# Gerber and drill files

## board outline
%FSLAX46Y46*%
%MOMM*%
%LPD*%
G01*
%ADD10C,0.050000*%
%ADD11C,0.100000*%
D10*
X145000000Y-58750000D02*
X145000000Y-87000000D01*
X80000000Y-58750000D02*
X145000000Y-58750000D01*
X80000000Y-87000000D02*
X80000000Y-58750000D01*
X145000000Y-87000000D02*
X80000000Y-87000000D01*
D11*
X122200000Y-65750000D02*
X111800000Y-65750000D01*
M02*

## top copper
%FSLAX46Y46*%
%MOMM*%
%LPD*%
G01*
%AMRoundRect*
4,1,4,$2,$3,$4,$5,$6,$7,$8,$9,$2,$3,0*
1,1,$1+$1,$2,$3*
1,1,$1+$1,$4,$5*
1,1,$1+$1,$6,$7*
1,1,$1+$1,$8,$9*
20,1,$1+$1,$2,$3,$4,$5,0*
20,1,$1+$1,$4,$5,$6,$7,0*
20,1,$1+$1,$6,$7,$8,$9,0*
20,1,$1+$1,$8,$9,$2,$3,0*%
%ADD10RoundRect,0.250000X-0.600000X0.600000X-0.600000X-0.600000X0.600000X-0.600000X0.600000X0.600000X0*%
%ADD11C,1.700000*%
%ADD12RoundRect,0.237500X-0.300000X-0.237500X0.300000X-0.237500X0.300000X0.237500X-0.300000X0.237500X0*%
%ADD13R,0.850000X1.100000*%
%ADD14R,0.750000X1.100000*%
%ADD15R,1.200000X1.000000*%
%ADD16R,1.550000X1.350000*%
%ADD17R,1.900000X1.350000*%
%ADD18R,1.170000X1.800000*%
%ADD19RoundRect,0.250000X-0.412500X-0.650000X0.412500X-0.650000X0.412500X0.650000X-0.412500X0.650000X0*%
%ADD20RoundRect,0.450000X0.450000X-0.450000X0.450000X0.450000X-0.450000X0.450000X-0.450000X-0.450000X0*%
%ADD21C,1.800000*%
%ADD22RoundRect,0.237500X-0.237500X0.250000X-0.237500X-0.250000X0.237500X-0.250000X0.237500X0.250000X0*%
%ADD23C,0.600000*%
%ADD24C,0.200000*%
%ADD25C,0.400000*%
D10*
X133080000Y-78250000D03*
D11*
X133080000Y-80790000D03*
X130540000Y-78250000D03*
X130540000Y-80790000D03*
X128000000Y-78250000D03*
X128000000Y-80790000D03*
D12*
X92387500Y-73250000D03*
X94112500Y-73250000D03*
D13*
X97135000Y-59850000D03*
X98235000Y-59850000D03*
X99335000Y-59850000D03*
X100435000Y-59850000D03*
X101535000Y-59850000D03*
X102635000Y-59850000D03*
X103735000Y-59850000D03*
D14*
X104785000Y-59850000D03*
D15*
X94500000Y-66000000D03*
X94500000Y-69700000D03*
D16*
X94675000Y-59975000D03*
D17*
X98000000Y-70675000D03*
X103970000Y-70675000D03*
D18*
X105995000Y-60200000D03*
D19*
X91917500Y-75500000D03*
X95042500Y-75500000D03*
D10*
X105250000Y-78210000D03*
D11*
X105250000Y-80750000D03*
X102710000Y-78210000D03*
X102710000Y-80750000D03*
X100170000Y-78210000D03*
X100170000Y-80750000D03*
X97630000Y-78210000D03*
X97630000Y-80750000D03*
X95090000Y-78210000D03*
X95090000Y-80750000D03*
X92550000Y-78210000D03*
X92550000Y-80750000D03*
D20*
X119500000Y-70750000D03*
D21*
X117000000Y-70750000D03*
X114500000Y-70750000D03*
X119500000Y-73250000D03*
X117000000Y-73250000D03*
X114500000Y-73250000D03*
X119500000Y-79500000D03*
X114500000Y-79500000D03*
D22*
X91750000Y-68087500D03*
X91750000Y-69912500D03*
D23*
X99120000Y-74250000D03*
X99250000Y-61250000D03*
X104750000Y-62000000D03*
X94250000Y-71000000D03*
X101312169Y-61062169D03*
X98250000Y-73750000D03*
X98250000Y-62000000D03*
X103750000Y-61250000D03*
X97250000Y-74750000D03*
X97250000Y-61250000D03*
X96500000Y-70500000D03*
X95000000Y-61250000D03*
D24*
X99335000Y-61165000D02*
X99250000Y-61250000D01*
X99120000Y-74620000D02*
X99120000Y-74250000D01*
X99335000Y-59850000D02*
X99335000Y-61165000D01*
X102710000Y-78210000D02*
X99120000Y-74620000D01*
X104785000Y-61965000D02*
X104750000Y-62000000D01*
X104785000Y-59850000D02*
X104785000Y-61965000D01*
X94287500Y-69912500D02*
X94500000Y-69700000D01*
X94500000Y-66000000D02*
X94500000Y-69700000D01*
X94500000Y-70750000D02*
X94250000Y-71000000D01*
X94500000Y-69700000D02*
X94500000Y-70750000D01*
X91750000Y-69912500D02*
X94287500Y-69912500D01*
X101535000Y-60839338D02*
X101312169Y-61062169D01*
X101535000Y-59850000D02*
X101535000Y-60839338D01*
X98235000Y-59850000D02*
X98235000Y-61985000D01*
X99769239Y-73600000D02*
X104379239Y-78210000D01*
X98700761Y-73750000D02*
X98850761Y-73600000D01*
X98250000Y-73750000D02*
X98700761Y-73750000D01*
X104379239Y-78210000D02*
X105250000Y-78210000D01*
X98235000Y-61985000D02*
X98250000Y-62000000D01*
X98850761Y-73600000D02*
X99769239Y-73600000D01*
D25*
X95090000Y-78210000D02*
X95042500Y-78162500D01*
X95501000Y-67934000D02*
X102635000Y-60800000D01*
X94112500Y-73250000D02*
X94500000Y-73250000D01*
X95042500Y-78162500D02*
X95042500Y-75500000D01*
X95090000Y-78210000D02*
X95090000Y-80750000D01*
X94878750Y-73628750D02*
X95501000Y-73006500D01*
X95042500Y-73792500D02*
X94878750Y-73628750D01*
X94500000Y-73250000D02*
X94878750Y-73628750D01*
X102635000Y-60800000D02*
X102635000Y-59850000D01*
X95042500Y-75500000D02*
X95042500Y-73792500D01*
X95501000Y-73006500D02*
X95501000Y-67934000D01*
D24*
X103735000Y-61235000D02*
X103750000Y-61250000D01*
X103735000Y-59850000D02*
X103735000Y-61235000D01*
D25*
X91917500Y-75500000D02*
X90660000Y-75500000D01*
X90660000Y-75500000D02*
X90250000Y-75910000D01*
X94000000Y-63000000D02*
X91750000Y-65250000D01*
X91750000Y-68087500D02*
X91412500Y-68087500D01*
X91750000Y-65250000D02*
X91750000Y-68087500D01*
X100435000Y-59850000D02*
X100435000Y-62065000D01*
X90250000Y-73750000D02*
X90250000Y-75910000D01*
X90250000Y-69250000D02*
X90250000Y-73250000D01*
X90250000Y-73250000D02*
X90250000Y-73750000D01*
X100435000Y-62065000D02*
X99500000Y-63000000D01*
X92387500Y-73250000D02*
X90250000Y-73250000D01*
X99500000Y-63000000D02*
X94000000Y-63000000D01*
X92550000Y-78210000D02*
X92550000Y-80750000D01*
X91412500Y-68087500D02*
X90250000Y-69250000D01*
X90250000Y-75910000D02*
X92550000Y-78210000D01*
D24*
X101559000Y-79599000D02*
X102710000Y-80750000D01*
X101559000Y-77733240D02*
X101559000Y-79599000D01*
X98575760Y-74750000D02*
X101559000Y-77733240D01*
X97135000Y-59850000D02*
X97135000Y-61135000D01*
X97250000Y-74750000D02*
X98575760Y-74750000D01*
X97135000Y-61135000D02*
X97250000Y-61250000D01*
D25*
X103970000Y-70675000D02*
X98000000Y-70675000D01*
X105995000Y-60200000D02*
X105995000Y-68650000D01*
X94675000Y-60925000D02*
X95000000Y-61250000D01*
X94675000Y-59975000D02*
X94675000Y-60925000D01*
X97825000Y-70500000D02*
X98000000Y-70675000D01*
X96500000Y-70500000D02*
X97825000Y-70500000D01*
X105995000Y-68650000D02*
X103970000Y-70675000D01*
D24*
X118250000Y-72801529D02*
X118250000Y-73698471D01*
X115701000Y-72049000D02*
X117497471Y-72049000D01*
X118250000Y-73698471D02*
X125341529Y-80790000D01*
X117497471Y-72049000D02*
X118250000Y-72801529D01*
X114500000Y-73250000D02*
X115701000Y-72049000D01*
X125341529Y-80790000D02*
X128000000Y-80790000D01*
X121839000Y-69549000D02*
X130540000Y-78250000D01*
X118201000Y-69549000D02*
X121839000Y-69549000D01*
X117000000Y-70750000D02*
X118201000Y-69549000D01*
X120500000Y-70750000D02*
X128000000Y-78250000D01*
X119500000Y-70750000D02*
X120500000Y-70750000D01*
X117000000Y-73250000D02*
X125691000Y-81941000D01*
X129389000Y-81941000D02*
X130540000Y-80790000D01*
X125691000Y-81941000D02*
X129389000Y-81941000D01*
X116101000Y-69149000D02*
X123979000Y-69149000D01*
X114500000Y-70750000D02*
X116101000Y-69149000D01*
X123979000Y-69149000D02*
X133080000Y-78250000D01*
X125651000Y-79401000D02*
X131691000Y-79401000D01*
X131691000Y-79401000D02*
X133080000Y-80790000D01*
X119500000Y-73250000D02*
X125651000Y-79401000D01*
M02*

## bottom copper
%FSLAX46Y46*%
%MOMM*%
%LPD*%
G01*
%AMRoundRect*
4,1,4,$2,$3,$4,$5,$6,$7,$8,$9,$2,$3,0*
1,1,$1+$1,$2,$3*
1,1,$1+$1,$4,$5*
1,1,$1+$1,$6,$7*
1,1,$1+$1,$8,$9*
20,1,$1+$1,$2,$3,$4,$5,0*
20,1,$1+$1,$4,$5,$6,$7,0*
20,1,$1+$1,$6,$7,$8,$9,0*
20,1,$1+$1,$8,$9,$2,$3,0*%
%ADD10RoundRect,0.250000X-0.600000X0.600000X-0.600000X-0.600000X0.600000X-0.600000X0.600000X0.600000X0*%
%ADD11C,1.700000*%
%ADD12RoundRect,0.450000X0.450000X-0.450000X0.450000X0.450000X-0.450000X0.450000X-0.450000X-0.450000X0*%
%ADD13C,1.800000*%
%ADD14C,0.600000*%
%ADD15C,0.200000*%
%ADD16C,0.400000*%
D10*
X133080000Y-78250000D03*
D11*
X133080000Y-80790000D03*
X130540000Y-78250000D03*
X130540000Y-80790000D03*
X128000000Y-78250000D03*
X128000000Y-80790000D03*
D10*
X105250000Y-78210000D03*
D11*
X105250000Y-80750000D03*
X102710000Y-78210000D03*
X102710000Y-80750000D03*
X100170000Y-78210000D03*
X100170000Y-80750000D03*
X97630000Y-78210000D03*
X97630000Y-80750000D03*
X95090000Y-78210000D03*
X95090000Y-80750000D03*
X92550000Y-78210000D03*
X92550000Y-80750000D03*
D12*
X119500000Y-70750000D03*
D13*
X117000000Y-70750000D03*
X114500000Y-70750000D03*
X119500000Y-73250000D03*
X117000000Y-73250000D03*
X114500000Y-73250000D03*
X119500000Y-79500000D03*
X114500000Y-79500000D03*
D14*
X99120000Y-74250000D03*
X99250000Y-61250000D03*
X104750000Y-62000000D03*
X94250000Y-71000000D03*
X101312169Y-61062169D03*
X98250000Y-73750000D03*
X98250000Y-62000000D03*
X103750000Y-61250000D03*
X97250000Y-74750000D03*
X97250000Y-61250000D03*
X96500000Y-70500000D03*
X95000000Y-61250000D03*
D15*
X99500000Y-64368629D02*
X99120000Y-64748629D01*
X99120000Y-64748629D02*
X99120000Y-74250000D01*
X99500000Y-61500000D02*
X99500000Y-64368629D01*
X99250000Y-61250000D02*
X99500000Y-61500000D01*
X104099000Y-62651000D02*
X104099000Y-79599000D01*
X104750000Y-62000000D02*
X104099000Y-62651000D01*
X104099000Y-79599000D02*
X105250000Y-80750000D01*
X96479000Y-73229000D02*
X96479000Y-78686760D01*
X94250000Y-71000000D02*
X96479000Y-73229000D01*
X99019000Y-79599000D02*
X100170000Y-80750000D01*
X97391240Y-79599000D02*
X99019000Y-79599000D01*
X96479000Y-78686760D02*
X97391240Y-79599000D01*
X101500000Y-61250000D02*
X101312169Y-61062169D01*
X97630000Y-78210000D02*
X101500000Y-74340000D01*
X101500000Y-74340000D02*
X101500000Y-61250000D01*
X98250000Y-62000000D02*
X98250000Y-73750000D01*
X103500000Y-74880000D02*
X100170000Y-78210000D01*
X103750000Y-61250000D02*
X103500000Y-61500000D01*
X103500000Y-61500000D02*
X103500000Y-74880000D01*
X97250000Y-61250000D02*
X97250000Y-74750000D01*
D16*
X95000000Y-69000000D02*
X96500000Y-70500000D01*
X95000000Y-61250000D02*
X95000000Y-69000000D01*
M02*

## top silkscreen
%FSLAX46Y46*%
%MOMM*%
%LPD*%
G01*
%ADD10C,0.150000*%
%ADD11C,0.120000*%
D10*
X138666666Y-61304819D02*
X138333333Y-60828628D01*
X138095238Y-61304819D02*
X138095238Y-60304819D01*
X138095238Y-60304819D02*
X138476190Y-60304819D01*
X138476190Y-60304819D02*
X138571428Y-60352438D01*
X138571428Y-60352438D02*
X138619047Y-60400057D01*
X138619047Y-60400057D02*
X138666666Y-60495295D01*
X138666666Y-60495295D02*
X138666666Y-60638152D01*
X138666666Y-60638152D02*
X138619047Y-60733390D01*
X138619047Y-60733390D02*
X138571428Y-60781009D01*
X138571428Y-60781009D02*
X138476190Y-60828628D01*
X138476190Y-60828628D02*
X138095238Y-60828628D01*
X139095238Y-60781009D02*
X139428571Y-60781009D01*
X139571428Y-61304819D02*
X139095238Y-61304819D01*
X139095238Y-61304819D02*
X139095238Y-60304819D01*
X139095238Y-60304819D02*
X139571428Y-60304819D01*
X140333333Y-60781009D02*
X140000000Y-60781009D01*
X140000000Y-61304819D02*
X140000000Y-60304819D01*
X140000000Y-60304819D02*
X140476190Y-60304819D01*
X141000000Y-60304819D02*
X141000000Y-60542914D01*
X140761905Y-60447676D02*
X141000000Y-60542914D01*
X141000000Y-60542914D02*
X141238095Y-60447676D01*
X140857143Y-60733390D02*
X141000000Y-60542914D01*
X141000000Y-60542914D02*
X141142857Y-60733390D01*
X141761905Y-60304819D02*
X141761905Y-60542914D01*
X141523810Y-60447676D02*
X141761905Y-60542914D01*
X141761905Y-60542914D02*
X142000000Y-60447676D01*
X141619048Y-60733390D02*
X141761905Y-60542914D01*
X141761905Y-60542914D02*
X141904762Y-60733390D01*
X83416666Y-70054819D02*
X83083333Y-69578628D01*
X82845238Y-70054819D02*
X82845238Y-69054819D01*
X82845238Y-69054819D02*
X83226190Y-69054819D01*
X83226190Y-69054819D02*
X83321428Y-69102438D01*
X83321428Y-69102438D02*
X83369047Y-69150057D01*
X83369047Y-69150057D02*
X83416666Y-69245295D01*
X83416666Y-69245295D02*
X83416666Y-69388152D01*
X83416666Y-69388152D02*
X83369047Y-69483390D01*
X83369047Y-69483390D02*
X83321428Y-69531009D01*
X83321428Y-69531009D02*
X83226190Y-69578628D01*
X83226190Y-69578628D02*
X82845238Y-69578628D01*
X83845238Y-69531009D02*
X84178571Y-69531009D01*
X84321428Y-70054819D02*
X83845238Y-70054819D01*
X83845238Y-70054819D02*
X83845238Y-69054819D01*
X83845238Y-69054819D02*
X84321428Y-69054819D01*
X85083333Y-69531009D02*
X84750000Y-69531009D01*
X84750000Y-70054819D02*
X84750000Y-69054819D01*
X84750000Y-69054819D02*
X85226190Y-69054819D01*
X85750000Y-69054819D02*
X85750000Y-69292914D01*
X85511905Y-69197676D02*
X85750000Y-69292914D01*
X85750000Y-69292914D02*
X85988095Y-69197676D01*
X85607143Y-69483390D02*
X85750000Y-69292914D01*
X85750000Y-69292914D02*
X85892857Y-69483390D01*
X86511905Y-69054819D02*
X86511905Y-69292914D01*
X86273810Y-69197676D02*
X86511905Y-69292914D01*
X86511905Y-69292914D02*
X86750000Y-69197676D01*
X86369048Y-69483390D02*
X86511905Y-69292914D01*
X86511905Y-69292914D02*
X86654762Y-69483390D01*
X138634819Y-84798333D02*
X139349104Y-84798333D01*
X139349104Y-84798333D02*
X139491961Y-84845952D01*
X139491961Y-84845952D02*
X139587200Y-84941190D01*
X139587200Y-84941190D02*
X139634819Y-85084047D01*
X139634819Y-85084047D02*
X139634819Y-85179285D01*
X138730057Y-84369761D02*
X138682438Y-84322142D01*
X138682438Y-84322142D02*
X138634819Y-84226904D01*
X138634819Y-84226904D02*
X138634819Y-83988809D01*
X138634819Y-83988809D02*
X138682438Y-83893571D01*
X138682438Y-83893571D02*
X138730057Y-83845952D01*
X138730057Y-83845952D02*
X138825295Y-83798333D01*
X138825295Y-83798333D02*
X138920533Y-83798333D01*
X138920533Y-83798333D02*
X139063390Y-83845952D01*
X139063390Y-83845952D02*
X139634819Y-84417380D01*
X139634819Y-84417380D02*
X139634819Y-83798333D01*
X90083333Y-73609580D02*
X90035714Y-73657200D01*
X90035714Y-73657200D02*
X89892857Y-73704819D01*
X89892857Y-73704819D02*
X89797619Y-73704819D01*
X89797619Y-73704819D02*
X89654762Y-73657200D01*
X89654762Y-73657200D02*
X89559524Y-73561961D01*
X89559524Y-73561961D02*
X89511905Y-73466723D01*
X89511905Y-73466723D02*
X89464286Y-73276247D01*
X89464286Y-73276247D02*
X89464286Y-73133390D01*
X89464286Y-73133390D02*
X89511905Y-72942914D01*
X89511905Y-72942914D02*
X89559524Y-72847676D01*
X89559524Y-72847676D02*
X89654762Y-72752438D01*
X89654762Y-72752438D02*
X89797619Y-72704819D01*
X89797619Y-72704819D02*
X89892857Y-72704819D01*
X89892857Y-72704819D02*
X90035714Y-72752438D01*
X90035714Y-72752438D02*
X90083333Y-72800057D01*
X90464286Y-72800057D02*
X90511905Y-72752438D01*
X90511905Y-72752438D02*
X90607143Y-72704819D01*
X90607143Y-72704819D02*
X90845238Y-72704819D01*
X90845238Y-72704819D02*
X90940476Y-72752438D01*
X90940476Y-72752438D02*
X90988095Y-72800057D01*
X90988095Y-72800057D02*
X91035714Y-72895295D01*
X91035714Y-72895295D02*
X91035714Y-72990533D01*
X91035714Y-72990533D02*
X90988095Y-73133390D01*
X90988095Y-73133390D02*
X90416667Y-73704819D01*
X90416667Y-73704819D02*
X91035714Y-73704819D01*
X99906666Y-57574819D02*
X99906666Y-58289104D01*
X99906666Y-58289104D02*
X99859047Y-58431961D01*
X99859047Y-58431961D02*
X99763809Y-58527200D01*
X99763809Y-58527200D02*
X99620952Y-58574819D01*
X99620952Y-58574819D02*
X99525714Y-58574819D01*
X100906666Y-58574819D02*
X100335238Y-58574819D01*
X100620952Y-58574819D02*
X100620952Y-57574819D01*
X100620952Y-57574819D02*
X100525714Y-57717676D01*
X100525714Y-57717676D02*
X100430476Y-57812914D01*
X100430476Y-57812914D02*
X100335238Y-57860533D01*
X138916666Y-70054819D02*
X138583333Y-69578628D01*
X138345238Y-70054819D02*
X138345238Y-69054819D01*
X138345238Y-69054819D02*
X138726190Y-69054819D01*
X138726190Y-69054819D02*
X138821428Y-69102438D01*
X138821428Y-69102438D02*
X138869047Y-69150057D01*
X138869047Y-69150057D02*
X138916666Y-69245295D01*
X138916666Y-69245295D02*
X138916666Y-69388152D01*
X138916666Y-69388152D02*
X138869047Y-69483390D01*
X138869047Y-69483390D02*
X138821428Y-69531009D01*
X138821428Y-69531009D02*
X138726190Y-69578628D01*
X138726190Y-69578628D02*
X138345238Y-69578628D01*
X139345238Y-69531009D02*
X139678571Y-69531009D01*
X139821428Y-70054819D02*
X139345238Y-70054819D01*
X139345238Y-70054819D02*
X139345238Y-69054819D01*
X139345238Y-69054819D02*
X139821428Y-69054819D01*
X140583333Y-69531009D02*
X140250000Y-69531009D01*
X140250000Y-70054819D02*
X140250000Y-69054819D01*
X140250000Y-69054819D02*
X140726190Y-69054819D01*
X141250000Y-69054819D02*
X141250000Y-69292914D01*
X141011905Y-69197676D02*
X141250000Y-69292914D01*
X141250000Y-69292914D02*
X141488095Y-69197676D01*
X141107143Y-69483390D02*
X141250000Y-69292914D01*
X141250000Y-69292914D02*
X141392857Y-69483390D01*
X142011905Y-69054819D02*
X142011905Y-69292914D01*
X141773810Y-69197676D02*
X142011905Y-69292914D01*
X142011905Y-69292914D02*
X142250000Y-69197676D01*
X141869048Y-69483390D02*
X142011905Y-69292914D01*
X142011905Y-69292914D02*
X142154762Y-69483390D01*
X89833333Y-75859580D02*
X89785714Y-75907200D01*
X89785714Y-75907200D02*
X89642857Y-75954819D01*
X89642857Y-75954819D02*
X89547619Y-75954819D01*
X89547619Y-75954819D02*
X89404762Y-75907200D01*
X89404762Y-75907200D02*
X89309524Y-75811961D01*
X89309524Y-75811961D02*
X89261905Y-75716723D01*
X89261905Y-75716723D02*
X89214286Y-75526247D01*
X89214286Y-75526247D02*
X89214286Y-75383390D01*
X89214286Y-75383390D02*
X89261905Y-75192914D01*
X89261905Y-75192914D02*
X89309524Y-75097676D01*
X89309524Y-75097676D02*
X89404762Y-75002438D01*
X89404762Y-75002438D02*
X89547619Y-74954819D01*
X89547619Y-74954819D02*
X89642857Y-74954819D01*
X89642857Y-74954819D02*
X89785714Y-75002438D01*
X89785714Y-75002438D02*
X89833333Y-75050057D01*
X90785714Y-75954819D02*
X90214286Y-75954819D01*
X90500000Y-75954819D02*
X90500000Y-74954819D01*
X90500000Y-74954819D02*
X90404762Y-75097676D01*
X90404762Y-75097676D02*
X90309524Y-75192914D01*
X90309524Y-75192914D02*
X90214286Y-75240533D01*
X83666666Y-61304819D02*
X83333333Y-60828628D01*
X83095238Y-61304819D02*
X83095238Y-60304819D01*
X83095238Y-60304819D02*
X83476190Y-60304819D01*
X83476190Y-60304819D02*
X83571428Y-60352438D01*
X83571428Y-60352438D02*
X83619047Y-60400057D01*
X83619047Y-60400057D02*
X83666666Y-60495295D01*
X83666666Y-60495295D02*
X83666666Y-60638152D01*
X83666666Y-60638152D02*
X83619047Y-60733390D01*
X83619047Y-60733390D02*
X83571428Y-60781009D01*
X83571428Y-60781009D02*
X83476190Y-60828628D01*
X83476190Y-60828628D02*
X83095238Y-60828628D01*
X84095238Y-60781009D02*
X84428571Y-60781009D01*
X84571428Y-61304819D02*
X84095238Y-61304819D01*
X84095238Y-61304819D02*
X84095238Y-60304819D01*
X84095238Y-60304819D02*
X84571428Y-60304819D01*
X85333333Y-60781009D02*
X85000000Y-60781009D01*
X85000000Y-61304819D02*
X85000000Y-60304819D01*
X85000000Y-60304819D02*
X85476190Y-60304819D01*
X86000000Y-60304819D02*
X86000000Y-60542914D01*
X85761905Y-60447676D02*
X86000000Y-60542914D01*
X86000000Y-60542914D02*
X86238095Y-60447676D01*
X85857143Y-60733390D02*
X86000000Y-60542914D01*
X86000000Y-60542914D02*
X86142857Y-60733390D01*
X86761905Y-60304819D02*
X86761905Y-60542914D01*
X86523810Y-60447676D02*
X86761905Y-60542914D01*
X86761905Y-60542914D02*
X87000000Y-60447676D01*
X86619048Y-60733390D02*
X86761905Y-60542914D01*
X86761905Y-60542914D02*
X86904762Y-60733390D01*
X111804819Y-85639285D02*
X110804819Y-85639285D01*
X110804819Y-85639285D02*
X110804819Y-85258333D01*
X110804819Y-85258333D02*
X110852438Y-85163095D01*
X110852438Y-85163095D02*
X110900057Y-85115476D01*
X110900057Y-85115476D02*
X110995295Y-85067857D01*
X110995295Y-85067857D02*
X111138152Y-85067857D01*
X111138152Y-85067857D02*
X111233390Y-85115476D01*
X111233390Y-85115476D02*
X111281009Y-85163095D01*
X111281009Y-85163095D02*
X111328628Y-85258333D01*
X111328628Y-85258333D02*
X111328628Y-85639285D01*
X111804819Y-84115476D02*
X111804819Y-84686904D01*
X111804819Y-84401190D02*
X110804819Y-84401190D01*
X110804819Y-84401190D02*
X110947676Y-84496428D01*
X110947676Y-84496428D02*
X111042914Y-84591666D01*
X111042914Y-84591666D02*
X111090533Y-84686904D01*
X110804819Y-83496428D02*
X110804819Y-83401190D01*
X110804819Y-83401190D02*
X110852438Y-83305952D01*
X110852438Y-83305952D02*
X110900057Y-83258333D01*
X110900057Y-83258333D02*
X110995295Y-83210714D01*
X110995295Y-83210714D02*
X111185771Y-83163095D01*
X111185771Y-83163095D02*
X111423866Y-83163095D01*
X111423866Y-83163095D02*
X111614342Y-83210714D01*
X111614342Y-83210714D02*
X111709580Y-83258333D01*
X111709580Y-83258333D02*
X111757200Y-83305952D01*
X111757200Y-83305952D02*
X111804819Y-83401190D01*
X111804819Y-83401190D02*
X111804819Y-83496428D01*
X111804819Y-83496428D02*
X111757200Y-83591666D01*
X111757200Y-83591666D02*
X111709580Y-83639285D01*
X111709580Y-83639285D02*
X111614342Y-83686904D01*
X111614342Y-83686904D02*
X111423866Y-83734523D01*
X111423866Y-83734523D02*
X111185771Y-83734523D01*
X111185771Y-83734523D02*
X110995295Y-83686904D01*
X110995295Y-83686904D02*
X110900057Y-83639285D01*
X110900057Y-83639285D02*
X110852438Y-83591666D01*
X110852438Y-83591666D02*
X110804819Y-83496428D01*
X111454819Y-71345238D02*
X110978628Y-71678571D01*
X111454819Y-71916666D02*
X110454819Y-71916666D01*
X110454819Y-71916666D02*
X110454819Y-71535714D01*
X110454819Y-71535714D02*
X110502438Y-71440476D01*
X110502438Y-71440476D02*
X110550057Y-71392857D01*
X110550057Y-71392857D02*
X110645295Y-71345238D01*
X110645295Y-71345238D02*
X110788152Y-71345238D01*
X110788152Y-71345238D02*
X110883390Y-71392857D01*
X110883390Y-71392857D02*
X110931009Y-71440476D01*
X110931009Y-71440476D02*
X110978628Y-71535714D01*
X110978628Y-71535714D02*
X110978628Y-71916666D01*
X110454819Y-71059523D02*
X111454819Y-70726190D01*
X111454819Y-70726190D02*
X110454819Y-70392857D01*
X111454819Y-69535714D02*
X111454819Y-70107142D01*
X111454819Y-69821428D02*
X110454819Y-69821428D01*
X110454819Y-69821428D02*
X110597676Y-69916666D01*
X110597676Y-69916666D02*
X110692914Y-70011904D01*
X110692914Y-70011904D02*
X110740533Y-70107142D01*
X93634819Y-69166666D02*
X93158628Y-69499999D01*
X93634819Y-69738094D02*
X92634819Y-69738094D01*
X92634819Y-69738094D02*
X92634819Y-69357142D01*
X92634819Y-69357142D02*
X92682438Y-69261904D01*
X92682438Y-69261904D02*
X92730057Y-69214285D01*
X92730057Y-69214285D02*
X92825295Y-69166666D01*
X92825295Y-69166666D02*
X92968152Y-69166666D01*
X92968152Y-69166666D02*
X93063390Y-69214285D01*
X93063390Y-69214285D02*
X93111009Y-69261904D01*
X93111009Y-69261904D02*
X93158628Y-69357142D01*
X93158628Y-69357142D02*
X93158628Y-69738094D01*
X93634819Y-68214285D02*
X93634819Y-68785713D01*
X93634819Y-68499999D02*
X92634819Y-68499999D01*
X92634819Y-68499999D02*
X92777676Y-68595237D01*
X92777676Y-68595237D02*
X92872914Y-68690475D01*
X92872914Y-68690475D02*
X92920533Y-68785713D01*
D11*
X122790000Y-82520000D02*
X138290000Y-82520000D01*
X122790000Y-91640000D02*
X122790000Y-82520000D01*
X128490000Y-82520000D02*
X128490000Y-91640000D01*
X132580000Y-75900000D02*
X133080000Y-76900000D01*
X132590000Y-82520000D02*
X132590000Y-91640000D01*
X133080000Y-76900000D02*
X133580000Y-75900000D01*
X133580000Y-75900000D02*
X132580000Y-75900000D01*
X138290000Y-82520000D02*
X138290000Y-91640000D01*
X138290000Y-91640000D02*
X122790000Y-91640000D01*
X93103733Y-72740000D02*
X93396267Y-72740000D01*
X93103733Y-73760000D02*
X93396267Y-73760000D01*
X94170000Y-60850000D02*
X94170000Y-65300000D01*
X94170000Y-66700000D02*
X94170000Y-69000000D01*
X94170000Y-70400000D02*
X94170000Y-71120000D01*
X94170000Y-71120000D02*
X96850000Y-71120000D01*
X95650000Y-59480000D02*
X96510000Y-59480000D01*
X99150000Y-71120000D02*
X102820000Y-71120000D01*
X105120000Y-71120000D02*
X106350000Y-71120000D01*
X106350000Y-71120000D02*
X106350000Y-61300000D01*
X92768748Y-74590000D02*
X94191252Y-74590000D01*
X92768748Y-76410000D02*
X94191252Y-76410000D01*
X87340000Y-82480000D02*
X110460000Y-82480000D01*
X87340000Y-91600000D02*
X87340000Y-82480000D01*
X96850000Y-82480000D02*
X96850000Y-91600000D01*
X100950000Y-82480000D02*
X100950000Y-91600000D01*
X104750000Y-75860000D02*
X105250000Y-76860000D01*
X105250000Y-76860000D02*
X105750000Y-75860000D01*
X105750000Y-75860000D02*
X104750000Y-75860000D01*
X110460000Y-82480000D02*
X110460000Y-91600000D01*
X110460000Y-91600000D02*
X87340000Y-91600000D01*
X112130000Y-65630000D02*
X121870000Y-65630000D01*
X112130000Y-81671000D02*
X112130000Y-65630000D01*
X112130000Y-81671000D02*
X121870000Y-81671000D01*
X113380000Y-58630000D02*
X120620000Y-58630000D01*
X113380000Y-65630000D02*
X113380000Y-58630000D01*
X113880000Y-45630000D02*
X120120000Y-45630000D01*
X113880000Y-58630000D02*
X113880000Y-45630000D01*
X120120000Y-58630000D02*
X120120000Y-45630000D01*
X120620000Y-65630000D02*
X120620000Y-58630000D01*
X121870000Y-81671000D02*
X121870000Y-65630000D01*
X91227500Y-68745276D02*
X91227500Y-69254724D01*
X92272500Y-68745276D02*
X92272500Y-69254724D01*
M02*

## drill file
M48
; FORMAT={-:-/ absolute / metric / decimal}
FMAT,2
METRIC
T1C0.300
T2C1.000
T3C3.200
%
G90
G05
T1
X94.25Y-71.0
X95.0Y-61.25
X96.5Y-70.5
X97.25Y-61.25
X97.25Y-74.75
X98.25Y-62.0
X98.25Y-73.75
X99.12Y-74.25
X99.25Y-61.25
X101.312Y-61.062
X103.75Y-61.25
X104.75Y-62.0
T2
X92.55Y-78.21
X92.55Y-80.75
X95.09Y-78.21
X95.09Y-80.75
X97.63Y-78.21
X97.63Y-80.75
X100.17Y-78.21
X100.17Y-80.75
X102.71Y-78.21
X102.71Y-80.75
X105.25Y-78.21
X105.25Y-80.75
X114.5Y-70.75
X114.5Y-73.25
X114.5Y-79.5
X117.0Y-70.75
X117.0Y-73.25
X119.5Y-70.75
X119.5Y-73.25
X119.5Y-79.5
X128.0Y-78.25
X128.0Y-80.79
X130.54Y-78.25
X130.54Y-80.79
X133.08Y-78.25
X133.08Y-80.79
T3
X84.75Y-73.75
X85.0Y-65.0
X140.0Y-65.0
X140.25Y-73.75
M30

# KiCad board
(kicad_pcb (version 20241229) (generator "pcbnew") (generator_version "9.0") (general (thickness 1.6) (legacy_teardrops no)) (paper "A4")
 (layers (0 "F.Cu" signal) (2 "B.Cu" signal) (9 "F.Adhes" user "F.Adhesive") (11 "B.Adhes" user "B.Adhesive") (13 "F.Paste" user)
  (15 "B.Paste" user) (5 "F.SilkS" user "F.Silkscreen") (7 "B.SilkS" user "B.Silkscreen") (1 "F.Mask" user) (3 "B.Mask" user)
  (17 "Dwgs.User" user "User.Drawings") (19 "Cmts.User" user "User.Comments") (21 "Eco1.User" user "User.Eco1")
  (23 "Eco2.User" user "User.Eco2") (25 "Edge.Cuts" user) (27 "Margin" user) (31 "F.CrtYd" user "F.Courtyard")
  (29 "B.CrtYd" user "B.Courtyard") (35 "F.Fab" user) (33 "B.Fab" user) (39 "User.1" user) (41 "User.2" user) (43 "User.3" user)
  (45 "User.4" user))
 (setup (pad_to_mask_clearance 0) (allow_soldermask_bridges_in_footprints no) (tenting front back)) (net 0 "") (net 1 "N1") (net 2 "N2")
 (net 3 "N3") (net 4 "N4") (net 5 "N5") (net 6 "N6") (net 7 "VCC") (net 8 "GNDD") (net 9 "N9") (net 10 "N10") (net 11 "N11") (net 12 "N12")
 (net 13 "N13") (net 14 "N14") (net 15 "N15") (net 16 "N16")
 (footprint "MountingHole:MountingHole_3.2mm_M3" (layer "F.Cu") (at 140 65)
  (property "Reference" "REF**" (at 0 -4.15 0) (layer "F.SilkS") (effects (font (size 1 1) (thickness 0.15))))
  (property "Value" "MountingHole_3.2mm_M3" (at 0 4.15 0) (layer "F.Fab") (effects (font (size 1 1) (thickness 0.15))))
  (pad "" np_thru_hole circle (at 0 0) (size 3.2 3.2) (drill 3.2) (layers "*.Cu" "*.Mask")))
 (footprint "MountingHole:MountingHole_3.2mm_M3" (layer "F.Cu") (at 84.75 73.75)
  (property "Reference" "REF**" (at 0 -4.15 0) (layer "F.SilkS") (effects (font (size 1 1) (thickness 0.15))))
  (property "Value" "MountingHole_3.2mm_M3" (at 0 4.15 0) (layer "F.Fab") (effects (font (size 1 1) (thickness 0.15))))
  (pad "" np_thru_hole circle (at 0 0) (size 3.2 3.2) (drill 3.2) (layers "*.Cu" "*.Mask")))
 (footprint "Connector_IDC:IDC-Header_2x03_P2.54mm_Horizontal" (layer "F.Cu") (at 133.08 78.25 -90)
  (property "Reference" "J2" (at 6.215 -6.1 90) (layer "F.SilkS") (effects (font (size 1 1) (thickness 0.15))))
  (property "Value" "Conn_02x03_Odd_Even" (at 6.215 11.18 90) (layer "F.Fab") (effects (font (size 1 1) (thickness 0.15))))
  (fp_line (start 4.27 10.29) (end 4.27 -5.21) (stroke (width 0.12) (type solid)) (layer "F.SilkS"))
  (fp_line (start 13.39 10.29) (end 4.27 10.29) (stroke (width 0.12) (type solid)) (layer "F.SilkS"))
  (fp_line (start 4.27 4.59) (end 13.39 4.59) (stroke (width 0.12) (type solid)) (layer "F.SilkS"))
  (fp_line (start -2.35 0.5) (end -1.35 0) (stroke (width 0.12) (type solid)) (layer "F.SilkS"))
  (fp_line (start 4.27 0.49) (end 13.39 0.49) (stroke (width 0.12) (type solid)) (layer "F.SilkS"))
  (fp_line (start -1.35 0) (end -2.35 -0.5) (stroke (width 0.12) (type solid)) (layer "F.SilkS"))
  (fp_line (start -2.35 -0.5) (end -2.35 0.5) (stroke (width 0.12) (type solid)) (layer "F.SilkS"))
  (fp_line (start 4.27 -5.21) (end 13.39 -5.21) (stroke (width 0.12) (type solid)) (layer "F.SilkS"))
  (fp_line (start 13.39 -5.21) (end 13.39 10.29) (stroke (width 0.12) (type solid)) (layer "F.SilkS"))
  (pad "1" thru_hole roundrect (at 0 0 270) (size 1.7 1.7) (drill 1) (layers "*.Cu" "*.Mask") (remove_unused_layers no)
   (roundrect_rratio 0.147059) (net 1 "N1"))
  (pad "2" thru_hole circle (at 2.54 0 270) (size 1.7 1.7) (drill 1) (layers "*.Cu" "*.Mask") (remove_unused_layers no) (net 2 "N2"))
  (pad "3" thru_hole circle (at 0 2.54 270) (size 1.7 1.7) (drill 1) (layers "*.Cu" "*.Mask") (remove_unused_layers no) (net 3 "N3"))
  (pad "4" thru_hole circle (at 2.54 2.54 270) (size 1.7 1.7) (drill 1) (layers "*.Cu" "*.Mask") (remove_unused_layers no) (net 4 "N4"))
  (pad "5" thru_hole circle (at 0 5.08 270) (size 1.7 1.7) (drill 1) (layers "*.Cu" "*.Mask") (remove_unused_layers no) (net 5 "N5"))
  (pad "6" thru_hole circle (at 2.54 5.08 270) (size 1.7 1.7) (drill 1) (layers "*.Cu" "*.Mask") (remove_unused_layers no) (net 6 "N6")))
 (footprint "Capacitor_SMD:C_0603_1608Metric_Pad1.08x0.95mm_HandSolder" (layer "F.Cu") (at 93.25 73.25)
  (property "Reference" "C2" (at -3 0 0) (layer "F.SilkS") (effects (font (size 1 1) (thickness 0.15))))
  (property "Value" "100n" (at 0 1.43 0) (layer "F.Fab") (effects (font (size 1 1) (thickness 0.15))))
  (fp_line (start -0.146267 -0.51) (end 0.146267 -0.51) (stroke (width 0.12) (type solid)) (layer "F.SilkS"))
  (fp_line (start -0.146267 0.51) (end 0.146267 0.51) (stroke (width 0.12) (type solid)) (layer "F.SilkS"))
  (pad "1" smd roundrect (at -0.8625 0) (size 1.075 0.95) (layers "F.Cu" "F.Mask" "F.Paste") (roundrect_rratio 0.25) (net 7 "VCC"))
  (pad "2" smd roundrect (at 0.8625 0) (size 1.075 0.95) (layers "F.Cu" "F.Mask" "F.Paste") (roundrect_rratio 0.25) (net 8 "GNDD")))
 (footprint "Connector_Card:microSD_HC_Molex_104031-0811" (layer "F.Cu") (at 100.24 65.3)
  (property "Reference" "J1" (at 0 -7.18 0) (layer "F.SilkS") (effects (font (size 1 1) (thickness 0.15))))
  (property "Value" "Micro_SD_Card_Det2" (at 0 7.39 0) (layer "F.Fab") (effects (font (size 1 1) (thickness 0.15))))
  (fp_line (start -6.07 -4.45) (end -6.07 0) (stroke (width 0.12) (type solid)) (layer "F.SilkS"))
  (fp_line (start -6.07 1.4) (end -6.07 3.7) (stroke (width 0.12) (type solid)) (layer "F.SilkS"))
  (fp_line (start -6.07 5.1) (end -6.07 5.82) (stroke (width 0.12) (type solid)) (layer "F.SilkS"))
  (fp_line (start -6.07 5.82) (end -3.39 5.82) (stroke (width 0.12) (type solid)) (layer "F.SilkS"))
  (fp_line (start -4.59 -5.82) (end -3.73 -5.82) (stroke (width 0.12) (type solid)) (layer "F.SilkS"))
  (fp_line (start -1.09 5.82) (end 2.58 5.82) (stroke (width 0.12) (type solid)) (layer "F.SilkS"))
  (fp_line (start 4.88 5.82) (end 6.11 5.82) (stroke (width 0.12) (type solid)) (layer "F.SilkS"))
  (fp_line (start 6.11 5.82) (end 6.11 -4) (stroke (width 0.12) (type solid)) (layer "F.SilkS"))
  (pad "1" smd rect (at -3.105 -5.45) (size 0.85 1.1) (layers "F.Cu" "F.Mask" "F.Paste") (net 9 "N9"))
  (pad "2" smd rect (at -2.005 -5.45) (size 0.85 1.1) (layers "F.Cu" "F.Mask" "F.Paste") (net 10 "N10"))
  (pad "3" smd rect (at -0.905 -5.45) (size 0.85 1.1) (layers "F.Cu" "F.Mask" "F.Paste") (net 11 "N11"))
  (pad "4" smd rect (at 0.195 -5.45) (size 0.85 1.1) (layers "F.Cu" "F.Mask" "F.Paste") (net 7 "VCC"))
  (pad "5" smd rect (at 1.295 -5.45) (size 0.85 1.1) (layers "F.Cu" "F.Mask" "F.Paste") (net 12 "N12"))
  (pad "6" smd rect (at 2.395 -5.45) (size 0.85 1.1) (layers "F.Cu" "F.Mask" "F.Paste") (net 8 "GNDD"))
  (pad "7" smd rect (at 3.495 -5.45) (size 0.85 1.1) (layers "F.Cu" "F.Mask" "F.Paste") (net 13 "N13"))
  (pad "8" smd rect (at 4.545 -5.45) (size 0.75 1.1) (layers "F.Cu" "F.Mask" "F.Paste") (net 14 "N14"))
  (pad "9" smd rect (at -5.74 0.7) (size 1.2 1) (layers "F.Cu" "F.Mask" "F.Paste") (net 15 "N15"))
  (pad "10" smd rect (at -5.74 4.4) (size 1.2 1) (layers "F.Cu" "F.Mask" "F.Paste") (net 15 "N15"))
  (pad "11" smd rect (at -5.565 -5.325) (size 1.55 1.35) (layers "F.Cu" "F.Mask" "F.Paste") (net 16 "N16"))
  (pad "11" smd rect (at -2.24 5.375) (size 1.9 1.35) (layers "F.Cu" "F.Mask" "F.Paste") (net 16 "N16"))
  (pad "11" smd rect (at 3.73 5.375) (size 1.9 1.35) (layers "F.Cu" "F.Mask" "F.Paste") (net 16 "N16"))
  (pad "11" smd rect (at 5.755 -5.1) (size 1.17 1.8) (layers "F.Cu" "F.Mask" "F.Paste") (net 16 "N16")))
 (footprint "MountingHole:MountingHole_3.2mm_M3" (layer "F.Cu") (at 140.25 73.75)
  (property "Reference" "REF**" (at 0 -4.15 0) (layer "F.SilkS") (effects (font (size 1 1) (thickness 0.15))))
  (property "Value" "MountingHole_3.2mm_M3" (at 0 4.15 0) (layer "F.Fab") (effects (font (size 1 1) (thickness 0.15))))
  (pad "" np_thru_hole circle (at 0 0) (size 3.2 3.2) (drill 3.2) (layers "*.Cu" "*.Mask")))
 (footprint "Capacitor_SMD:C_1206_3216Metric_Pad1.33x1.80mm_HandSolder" (layer "F.Cu") (at 93.48 75.5)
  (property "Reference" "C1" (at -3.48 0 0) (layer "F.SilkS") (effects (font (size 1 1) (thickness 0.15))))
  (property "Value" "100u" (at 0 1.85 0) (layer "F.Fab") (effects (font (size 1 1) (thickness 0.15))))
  (fp_line (start -0.711252 -0.91) (end 0.711252 -0.91) (stroke (width 0.12) (type solid)) (layer "F.SilkS"))
  (fp_line (start -0.711252 0.91) (end 0.711252 0.91) (stroke (width 0.12) (type solid)) (layer "F.SilkS"))
  (pad "1" smd roundrect (at -1.5625 0) (size 1.325 1.8) (layers "F.Cu" "F.Mask" "F.Paste") (roundrect_rratio 0.188679) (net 7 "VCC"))
  (pad "2" smd roundrect (at 1.5625 0) (size 1.325 1.8) (layers "F.Cu" "F.Mask" "F.Paste") (roundrect_rratio 0.188679) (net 8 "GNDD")))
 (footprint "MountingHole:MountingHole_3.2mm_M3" (layer "F.Cu") (at 85 65)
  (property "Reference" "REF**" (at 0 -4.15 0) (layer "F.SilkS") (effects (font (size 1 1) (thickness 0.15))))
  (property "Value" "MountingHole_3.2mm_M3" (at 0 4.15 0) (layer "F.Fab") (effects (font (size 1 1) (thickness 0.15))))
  (pad "" np_thru_hole circle (at 0 0) (size 3.2 3.2) (drill 3.2) (layers "*.Cu" "*.Mask")))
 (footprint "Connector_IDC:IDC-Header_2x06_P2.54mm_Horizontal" (layer "F.Cu") (at 105.25 78.21 -90)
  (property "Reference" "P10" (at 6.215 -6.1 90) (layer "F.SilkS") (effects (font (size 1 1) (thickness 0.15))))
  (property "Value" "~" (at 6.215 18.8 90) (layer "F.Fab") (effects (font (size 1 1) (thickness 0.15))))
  (fp_line (start 4.27 17.91) (end 4.27 -5.21) (stroke (width 0.12) (type solid)) (layer "F.SilkS"))
  (fp_line (start 13.39 17.91) (end 4.27 17.91) (stroke (width 0.12) (type solid)) (layer "F.SilkS"))
  (fp_line (start 4.27 8.4) (end 13.39 8.4) (stroke (width 0.12) (type solid)) (layer "F.SilkS"))
  (fp_line (start 4.27 4.3) (end 13.39 4.3) (stroke (width 0.12) (type solid)) (layer "F.SilkS"))
  (fp_line (start -2.35 0.5) (end -1.35 0) (stroke (width 0.12) (type solid)) (layer "F.SilkS"))
  (fp_line (start -1.35 0) (end -2.35 -0.5) (stroke (width 0.12) (type solid)) (layer "F.SilkS"))
  (fp_line (start -2.35 -0.5) (end -2.35 0.5) (stroke (width 0.12) (type solid)) (layer "F.SilkS"))
  (fp_line (start 4.27 -5.21) (end 13.39 -5.21) (stroke (width 0.12) (type solid)) (layer "F.SilkS"))
  (fp_line (start 13.39 -5.21) (end 13.39 17.91) (stroke (width 0.12) (type solid)) (layer "F.SilkS"))
  (pad "1" thru_hole roundrect (at 0 0 270) (size 1.7 1.7) (drill 1) (layers "*.Cu" "*.Mask") (remove_unused_layers no)
   (roundrect_rratio 0.147059) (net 10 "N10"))
  (pad "2" thru_hole circle (at 2.54 0 270) (size 1.7 1.7) (drill 1) (layers "*.Cu" "*.Mask") (remove_unused_layers no) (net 14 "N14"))
  (pad "3" thru_hole circle (at 0 2.54 270) (size 1.7 1.7) (drill 1) (layers "*.Cu" "*.Mask") (remove_unused_layers no) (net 11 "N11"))
  (pad "4" thru_hole circle (at 2.54 2.54 270) (size 1.7 1.7) (drill 1) (layers "*.Cu" "*.Mask") (remove_unused_layers no) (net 9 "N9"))
  (pad "5" thru_hole circle (at 0 5.08 270) (size 1.7 1.7) (drill 1) (layers "*.Cu" "*.Mask") (remove_unused_layers no) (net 13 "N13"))
  (pad "6" thru_hole circle (at 2.54 5.08 270) (size 1.7 1.7) (drill 1) (layers "*.Cu" "*.Mask") (remove_unused_layers no) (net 15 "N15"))
  (pad "7" thru_hole circle (at 0 7.62 270) (size 1.7 1.7) (drill 1) (layers "*.Cu" "*.Mask") (remove_unused_layers no) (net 12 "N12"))
  (pad "8" thru_hole circle (at 2.54 7.62 270) (size 1.7 1.7) (drill 1) (layers "*.Cu" "*.Mask") (remove_unused_layers no))
  (pad "9" thru_hole circle (at 0 10.16 270) (size 1.7 1.7) (drill 1) (layers "*.Cu" "*.Mask") (remove_unused_layers no) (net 8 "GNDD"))
  (pad "10" thru_hole circle (at 2.54 10.16 270) (size 1.7 1.7) (drill 1) (layers "*.Cu" "*.Mask") (remove_unused_layers no) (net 8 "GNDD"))
  (pad "11" thru_hole circle (at 0 12.7 270) (size 1.7 1.7) (drill 1) (layers "*.Cu" "*.Mask") (remove_unused_layers no) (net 7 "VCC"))
  (pad "12" thru_hole circle (at 2.54 12.7 270) (size 1.7 1.7) (drill 1) (layers "*.Cu" "*.Mask") (remove_unused_layers no) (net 7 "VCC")))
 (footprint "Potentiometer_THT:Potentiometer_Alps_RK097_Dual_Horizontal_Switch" (layer "F.Cu") (at 119.5 70.75 -90)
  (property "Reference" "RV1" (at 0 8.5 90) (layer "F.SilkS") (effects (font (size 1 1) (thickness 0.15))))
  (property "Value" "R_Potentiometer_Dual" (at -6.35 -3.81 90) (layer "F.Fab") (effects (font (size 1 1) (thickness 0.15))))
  (fp_line (start -5.12 7.37) (end -5.12 -2.37) (stroke (width 0.12) (type solid)) (layer "F.SilkS"))
  (fp_line (start 10.921 7.37) (end -5.12 7.37) (stroke (width 0.12) (type solid)) (layer "F.SilkS"))
  (fp_line (start 10.921 7.37) (end 10.921 -2.37) (stroke (width 0.12) (type solid)) (layer "F.SilkS"))
  (fp_line (start -12.12 6.12) (end -12.12 -1.12) (stroke (width 0.12) (type solid)) (layer "F.SilkS"))
  (fp_line (start -5.12 6.12) (end -12.12 6.12) (stroke (width 0.12) (type solid)) (layer "F.SilkS"))
  (fp_line (start -25.12 5.62) (end -25.12 -0.62) (stroke (width 0.12) (type solid)) (layer "F.SilkS"))
  (fp_line (start -12.12 5.62) (end -25.12 5.62) (stroke (width 0.12) (type solid)) (layer "F.SilkS"))
  (fp_line (start -12.12 -0.62) (end -25.12 -0.62) (stroke (width 0.12) (type solid)) (layer "F.SilkS"))
  (fp_line (start -5.12 -1.12) (end -12.12 -1.12) (stroke (width 0.12) (type solid)) (layer "F.SilkS"))
  (fp_line (start 10.921 -2.37) (end -5.12 -2.37) (stroke (width 0.12) (type solid)) (layer "F.SilkS"))
  (fp_line (start -5 -2.7) (end -5 7.7) (stroke (width 0.1) (type solid)) (layer "Edge.Cuts"))
  (pad "1" thru_hole roundrect (at 0 0 90) (size 1.8 1.8) (drill 1) (layers "*.Cu" "*.Mask") (remove_unused_layers no)
   (roundrect_rratio 0.25) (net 5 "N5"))
  (pad "2" thru_hole circle (at 0 2.5 90) (size 1.8 1.8) (drill 1) (layers "*.Cu" "*.Mask") (remove_unused_layers no) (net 3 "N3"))
  (pad "3" thru_hole circle (at 0 5 90) (size 1.8 1.8) (drill 1) (layers "*.Cu" "*.Mask") (remove_unused_layers no) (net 1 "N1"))
  (pad "4" thru_hole circle (at 2.5 0 90) (size 1.8 1.8) (drill 1) (layers "*.Cu" "*.Mask") (remove_unused_layers no) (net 2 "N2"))
  (pad "5" thru_hole circle (at 2.5 2.5 90) (size 1.8 1.8) (drill 1) (layers "*.Cu" "*.Mask") (remove_unused_layers no) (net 4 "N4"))
  (pad "6" thru_hole circle (at 2.5 5 90) (size 1.8 1.8) (drill 1) (layers "*.Cu" "*.Mask") (remove_unused_layers no) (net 6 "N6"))
  (pad "7" thru_hole circle (at 8.75 0 90) (size 1.8 1.8) (drill 1) (layers "*.Cu" "*.Mask") (remove_unused_layers no))
  (pad "8" thru_hole circle (at 8.75 5 90) (size 1.8 1.8) (drill 1) (layers "*.Cu" "*.Mask") (remove_unused_layers no)))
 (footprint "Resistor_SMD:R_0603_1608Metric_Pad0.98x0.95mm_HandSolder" (layer "F.Cu") (at 91.75 69 -90)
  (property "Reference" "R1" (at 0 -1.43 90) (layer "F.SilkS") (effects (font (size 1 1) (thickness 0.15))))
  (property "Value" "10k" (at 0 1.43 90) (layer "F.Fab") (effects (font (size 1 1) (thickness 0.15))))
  (fp_line (start -0.254724 0.5225) (end 0.254724 0.5225) (stroke (width 0.12) (type solid)) (layer "F.SilkS"))
  (fp_line (start -0.254724 -0.5225) (end 0.254724 -0.5225) (stroke (width 0.12) (type solid)) (layer "F.SilkS"))
  (pad "1" smd roundrect (at -0.9125 0 270) (size 0.975 0.95) (layers "F.Cu" "F.Mask" "F.Paste") (roundrect_rratio 0.25) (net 7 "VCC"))
  (pad "2" smd roundrect (at 0.9125 0 270) (size 0.975 0.95) (layers "F.Cu" "F.Mask" "F.Paste") (roundrect_rratio 0.25) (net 15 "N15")))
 (gr_line (start 145 58.75) (end 145 87) (stroke (width 0.05) (type default)) (layer "Edge.Cuts"))
 (gr_line (start 80 58.75) (end 145 58.75) (stroke (width 0.05) (type default)) (layer "Edge.Cuts"))
 (gr_line (start 80 87) (end 80 58.75) (stroke (width 0.05) (type default)) (layer "Edge.Cuts"))
 (gr_line (start 145 87) (end 80 87) (stroke (width 0.05) (type default)) (layer "Edge.Cuts"))
 (segment (start 99.335 61.165) (end 99.25 61.25) (width 0.2) (layer "F.Cu") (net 11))
 (segment (start 99.12 74.62) (end 99.12 74.25) (width 0.2) (layer "F.Cu") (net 11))
 (segment (start 99.335 59.85) (end 99.335 61.165) (width 0.2) (layer "F.Cu") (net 11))
 (segment (start 102.71 78.21) (end 99.12 74.62) (width 0.2) (layer "F.Cu") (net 11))
 (via (at 99.12 74.25) (size 0.6) (drill 0.3) (layers "F.Cu" "B.Cu") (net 11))
 (via (at 99.25 61.25) (size 0.6) (drill 0.3) (layers "F.Cu" "B.Cu") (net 11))
 (segment (start 99.5 64.368629) (end 99.12 64.748629) (width 0.2) (layer "B.Cu") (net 11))
 (segment (start 99.12 64.748629) (end 99.12 74.25) (width 0.2) (layer "B.Cu") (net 11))
 (segment (start 99.5 61.5) (end 99.5 64.368629) (width 0.2) (layer "B.Cu") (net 11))
 (segment (start 99.25 61.25) (end 99.5 61.5) (width 0.2) (layer "B.Cu") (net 11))
 (segment (start 104.785 61.965) (end 104.75 62) (width 0.2) (layer "F.Cu") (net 14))
 (segment (start 104.785 59.85) (end 104.785 61.965) (width 0.2) (layer "F.Cu") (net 14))
 (via (at 104.75 62) (size 0.6) (drill 0.3) (layers "F.Cu" "B.Cu") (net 14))
 (segment (start 104.099 62.651) (end 104.099 79.599) (width 0.2) (layer "B.Cu") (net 14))
 (segment (start 104.75 62) (end 104.099 62.651) (width 0.2) (layer "B.Cu") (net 14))
 (segment (start 104.099 79.599) (end 105.25 80.75) (width 0.2) (layer "B.Cu") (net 14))
 (segment (start 94.2875 69.9125) (end 94.5 69.7) (width 0.2) (layer "F.Cu") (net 15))
 (segment (start 94.5 66) (end 94.5 69.7) (width 0.2) (layer "F.Cu") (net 15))
 (segment (start 94.5 70.75) (end 94.25 71) (width 0.2) (layer "F.Cu") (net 15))
 (segment (start 94.5 69.7) (end 94.5 70.75) (width 0.2) (layer "F.Cu") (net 15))
 (segment (start 91.75 69.9125) (end 94.2875 69.9125) (width 0.2) (layer "F.Cu") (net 15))
 (via (at 94.25 71) (size 0.6) (drill 0.3) (layers "F.Cu" "B.Cu") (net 15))
 (segment (start 96.479 73.229) (end 96.479 78.68676) (width 0.2) (layer "B.Cu") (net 15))
 (segment (start 94.25 71) (end 96.479 73.229) (width 0.2) (layer "B.Cu") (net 15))
 (segment (start 99.019 79.599) (end 100.17 80.75) (width 0.2) (layer "B.Cu") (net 15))
 (segment (start 97.39124 79.599) (end 99.019 79.599) (width 0.2) (layer "B.Cu") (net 15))
 (segment (start 96.479 78.68676) (end 97.39124 79.599) (width 0.2) (layer "B.Cu") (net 15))
 (segment (start 101.535 60.839338) (end 101.312169 61.062169) (width 0.2) (layer "F.Cu") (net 12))
 (segment (start 101.535 59.85) (end 101.535 60.839338) (width 0.2) (layer "F.Cu") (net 12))
 (via (at 101.312169 61.062169) (size 0.6) (drill 0.3) (layers "F.Cu" "B.Cu") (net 12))
 (segment (start 101.5 61.25) (end 101.312169 61.062169) (width 0.2) (layer "B.Cu") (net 12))
 (segment (start 97.63 78.21) (end 101.5 74.34) (width 0.2) (layer "B.Cu") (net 12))
 (segment (start 101.5 74.34) (end 101.5 61.25) (width 0.2) (layer "B.Cu") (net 12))
 (segment (start 98.235 59.85) (end 98.235 61.985) (width 0.2) (layer "F.Cu") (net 10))
 (segment (start 99.769239 73.6) (end 104.379239 78.21) (width 0.2) (layer "F.Cu") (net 10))
 (segment (start 98.700761 73.75) (end 98.850761 73.6) (width 0.2) (layer "F.Cu") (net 10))
 (segment (start 98.25 73.75) (end 98.700761 73.75) (width 0.2) (layer "F.Cu") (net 10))
 (segment (start 104.379239 78.21) (end 105.25 78.21) (width 0.2) (layer "F.Cu") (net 10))
 (segment (start 98.235 61.985) (end 98.25 62) (width 0.2) (layer "F.Cu") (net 10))
 (segment (start 98.850761 73.6) (end 99.769239 73.6) (width 0.2) (layer "F.Cu") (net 10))
 (via (at 98.25 73.75) (size 0.6) (drill 0.3) (layers "F.Cu" "B.Cu") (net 10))
 (via (at 98.25 62) (size 0.6) (drill 0.3) (layers "F.Cu" "B.Cu") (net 10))
 (segment (start 98.25 62) (end 98.25 73.75) (width 0.2) (layer "B.Cu") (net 10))
 (segment (start 95.09 78.21) (end 95.0425 78.1625) (width 0.4) (layer "F.Cu") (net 8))
 (segment (start 95.501 67.934) (end 102.635 60.8) (width 0.4) (layer "F.Cu") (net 8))
 (segment (start 94.1125 73.25) (end 94.5 73.25) (width 0.4) (layer "F.Cu") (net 8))
 (segment (start 95.0425 78.1625) (end 95.0425 75.5) (width 0.4) (layer "F.Cu") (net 8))
 (segment (start 95.09 78.21) (end 95.09 80.75) (width 0.4) (layer "F.Cu") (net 8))
 (segment (start 94.87875 73.62875) (end 95.501 73.0065) (width 0.4) (layer "F.Cu") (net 8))
 (segment (start 95.0425 73.7925) (end 94.87875 73.62875) (width 0.4) (layer "F.Cu") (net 8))
 (segment (start 94.5 73.25) (end 94.87875 73.62875) (width 0.4) (layer "F.Cu") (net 8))
 (segment (start 102.635 60.8) (end 102.635 59.85) (width 0.4) (layer "F.Cu") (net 8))
 (segment (start 95.0425 75.5) (end 95.0425 73.7925) (width 0.4) (layer "F.Cu") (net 8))
 (segment (start 95.501 73.0065) (end 95.501 67.934) (width 0.4) (layer "F.Cu") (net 8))
 (segment (start 103.735 61.235) (end 103.75 61.25) (width 0.2) (layer "F.Cu") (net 13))
 (segment (start 103.735 59.85) (end 103.735 61.235) (width 0.2) (layer "F.Cu") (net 13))
 (via (at 103.75 61.25) (size 0.6) (drill 0.3) (layers "F.Cu" "B.Cu") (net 13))
 (segment (start 103.5 74.88) (end 100.17 78.21) (width 0.2) (layer "B.Cu") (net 13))
 (segment (start 103.75 61.25) (end 103.5 61.5) (width 0.2) (layer "B.Cu") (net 13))
 (segment (start 103.5 61.5) (end 103.5 74.88) (width 0.2) (layer "B.Cu") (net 13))
 (segment (start 91.9175 75.5) (end 90.66 75.5) (width 0.4) (layer "F.Cu") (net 7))
 (segment (start 90.66 75.5) (end 90.25 75.91) (width 0.4) (layer "F.Cu") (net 7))
 (segment (start 94 63) (end 91.75 65.25) (width 0.4) (layer "F.Cu") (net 7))
 (segment (start 91.75 68.0875) (end 91.4125 68.0875) (width 0.4) (layer "F.Cu") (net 7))
 (segment (start 91.75 65.25) (end 91.75 68.0875) (width 0.4) (layer "F.Cu") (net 7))
 (segment (start 100.435 59.85) (end 100.435 62.065) (width 0.4) (layer "F.Cu") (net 7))
 (segment (start 90.25 73.75) (end 90.25 75.91) (width 0.4) (layer "F.Cu") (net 7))
 (segment (start 90.25 69.25) (end 90.25 73.25) (width 0.4) (layer "F.Cu") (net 7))
 (segment (start 90.25 73.25) (end 90.25 73.75) (width 0.4) (layer "F.Cu") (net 7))
 (segment (start 100.435 62.065) (end 99.5 63) (width 0.4) (layer "F.Cu") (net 7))
 (segment (start 92.3875 73.25) (end 90.25 73.25) (width 0.4) (layer "F.Cu") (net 7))
 (segment (start 99.5 63) (end 94 63) (width 0.4) (layer "F.Cu") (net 7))
 (segment (start 92.55 78.21) (end 92.55 80.75) (width 0.4) (layer "F.Cu") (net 7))
 (segment (start 91.4125 68.0875) (end 90.25 69.25) (width 0.4) (layer "F.Cu") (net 7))
 (segment (start 90.25 75.91) (end 92.55 78.21) (width 0.4) (layer "F.Cu") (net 7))
 (segment (start 101.559 79.599) (end 102.71 80.75) (width 0.2) (layer "F.Cu") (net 9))
 (segment (start 101.559 77.73324) (end 101.559 79.599) (width 0.2) (layer "F.Cu") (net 9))
 (segment (start 98.57576 74.75) (end 101.559 77.73324) (width 0.2) (layer "F.Cu") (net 9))
 (segment (start 97.135 59.85) (end 97.135 61.135) (width 0.2) (layer "F.Cu") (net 9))
 (segment (start 97.25 74.75) (end 98.57576 74.75) (width 0.2) (layer "F.Cu") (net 9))
 (segment (start 97.135 61.135) (end 97.25 61.25) (width 0.2) (layer "F.Cu") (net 9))
 (via (at 97.25 74.75) (size 0.6) (drill 0.3) (layers "F.Cu" "B.Cu") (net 9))
 (via (at 97.25 61.25) (size 0.6) (drill 0.3) (layers "F.Cu" "B.Cu") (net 9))
 (segment (start 97.25 61.25) (end 97.25 74.75) (width 0.2) (layer "B.Cu") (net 9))
 (segment (start 103.97 70.675) (end 98 70.675) (width 0.4) (layer "F.Cu") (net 16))
 (segment (start 105.995 60.2) (end 105.995 68.65) (width 0.4) (layer "F.Cu") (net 16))
 (segment (start 94.675 60.925) (end 95 61.25) (width 0.4) (layer "F.Cu") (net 16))
 (segment (start 94.675 59.975) (end 94.675 60.925) (width 0.4) (layer "F.Cu") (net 16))
 (segment (start 97.825 70.5) (end 98 70.675) (width 0.4) (layer "F.Cu") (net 16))
 (segment (start 96.5 70.5) (end 97.825 70.5) (width 0.4) (layer "F.Cu") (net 16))
 (segment (start 105.995 68.65) (end 103.97 70.675) (width 0.4) (layer "F.Cu") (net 16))
 (via (at 96.5 70.5) (size 0.6) (drill 0.3) (layers "F.Cu" "B.Cu") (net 16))
 (via (at 95 61.25) (size 0.6) (drill 0.3) (layers "F.Cu" "B.Cu") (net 16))
 (segment (start 95 69) (end 96.5 70.5) (width 0.4) (layer "B.Cu") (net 16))
 (segment (start 95 61.25) (end 95 69) (width 0.4) (layer "B.Cu") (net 16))
 (segment (start 118.25 72.801529) (end 118.25 73.698471) (width 0.2) (layer "F.Cu") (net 6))
 (segment (start 115.701 72.049) (end 117.497471 72.049) (width 0.2) (layer "F.Cu") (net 6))
 (segment (start 118.25 73.698471) (end 125.341529 80.79) (width 0.2) (layer "F.Cu") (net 6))
 (segment (start 117.497471 72.049) (end 118.25 72.801529) (width 0.2) (layer "F.Cu") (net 6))
 (segment (start 114.5 73.25) (end 115.701 72.049) (width 0.2) (layer "F.Cu") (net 6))
 (segment (start 125.341529 80.79) (end 128 80.79) (width 0.2) (layer "F.Cu") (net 6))
 (segment (start 121.839 69.549) (end 130.54 78.25) (width 0.2) (layer "F.Cu") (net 3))
 (segment (start 118.201 69.549) (end 121.839 69.549) (width 0.2) (layer "F.Cu") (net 3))
 (segment (start 117 70.75) (end 118.201 69.549) (width 0.2) (layer "F.Cu") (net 3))
 (segment (start 120.5 70.75) (end 128 78.25) (width 0.2) (layer "F.Cu") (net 5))
 (segment (start 119.5 70.75) (end 120.5 70.75) (width 0.2) (layer "F.Cu") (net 5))
 (segment (start 117 73.25) (end 125.691 81.941) (width 0.2) (layer "F.Cu") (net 4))
 (segment (start 129.389 81.941) (end 130.54 80.79) (width 0.2) (layer "F.Cu") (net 4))
 (segment (start 125.691 81.941) (end 129.389 81.941) (width 0.2) (layer "F.Cu") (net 4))
 (segment (start 116.101 69.149) (end 123.979 69.149) (width 0.2) (layer "F.Cu") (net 1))
 (segment (start 114.5 70.75) (end 116.101 69.149) (width 0.2) (layer "F.Cu") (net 1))
 (segment (start 123.979 69.149) (end 133.08 78.25) (width 0.2) (layer "F.Cu") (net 1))
 (segment (start 125.651 79.401) (end 131.691 79.401) (width 0.2) (layer "F.Cu") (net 2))
 (segment (start 131.691 79.401) (end 133.08 80.79) (width 0.2) (layer "F.Cu") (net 2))
 (segment (start 119.5 73.25) (end 125.651 79.401) (width 0.2) (layer "F.Cu") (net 2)))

